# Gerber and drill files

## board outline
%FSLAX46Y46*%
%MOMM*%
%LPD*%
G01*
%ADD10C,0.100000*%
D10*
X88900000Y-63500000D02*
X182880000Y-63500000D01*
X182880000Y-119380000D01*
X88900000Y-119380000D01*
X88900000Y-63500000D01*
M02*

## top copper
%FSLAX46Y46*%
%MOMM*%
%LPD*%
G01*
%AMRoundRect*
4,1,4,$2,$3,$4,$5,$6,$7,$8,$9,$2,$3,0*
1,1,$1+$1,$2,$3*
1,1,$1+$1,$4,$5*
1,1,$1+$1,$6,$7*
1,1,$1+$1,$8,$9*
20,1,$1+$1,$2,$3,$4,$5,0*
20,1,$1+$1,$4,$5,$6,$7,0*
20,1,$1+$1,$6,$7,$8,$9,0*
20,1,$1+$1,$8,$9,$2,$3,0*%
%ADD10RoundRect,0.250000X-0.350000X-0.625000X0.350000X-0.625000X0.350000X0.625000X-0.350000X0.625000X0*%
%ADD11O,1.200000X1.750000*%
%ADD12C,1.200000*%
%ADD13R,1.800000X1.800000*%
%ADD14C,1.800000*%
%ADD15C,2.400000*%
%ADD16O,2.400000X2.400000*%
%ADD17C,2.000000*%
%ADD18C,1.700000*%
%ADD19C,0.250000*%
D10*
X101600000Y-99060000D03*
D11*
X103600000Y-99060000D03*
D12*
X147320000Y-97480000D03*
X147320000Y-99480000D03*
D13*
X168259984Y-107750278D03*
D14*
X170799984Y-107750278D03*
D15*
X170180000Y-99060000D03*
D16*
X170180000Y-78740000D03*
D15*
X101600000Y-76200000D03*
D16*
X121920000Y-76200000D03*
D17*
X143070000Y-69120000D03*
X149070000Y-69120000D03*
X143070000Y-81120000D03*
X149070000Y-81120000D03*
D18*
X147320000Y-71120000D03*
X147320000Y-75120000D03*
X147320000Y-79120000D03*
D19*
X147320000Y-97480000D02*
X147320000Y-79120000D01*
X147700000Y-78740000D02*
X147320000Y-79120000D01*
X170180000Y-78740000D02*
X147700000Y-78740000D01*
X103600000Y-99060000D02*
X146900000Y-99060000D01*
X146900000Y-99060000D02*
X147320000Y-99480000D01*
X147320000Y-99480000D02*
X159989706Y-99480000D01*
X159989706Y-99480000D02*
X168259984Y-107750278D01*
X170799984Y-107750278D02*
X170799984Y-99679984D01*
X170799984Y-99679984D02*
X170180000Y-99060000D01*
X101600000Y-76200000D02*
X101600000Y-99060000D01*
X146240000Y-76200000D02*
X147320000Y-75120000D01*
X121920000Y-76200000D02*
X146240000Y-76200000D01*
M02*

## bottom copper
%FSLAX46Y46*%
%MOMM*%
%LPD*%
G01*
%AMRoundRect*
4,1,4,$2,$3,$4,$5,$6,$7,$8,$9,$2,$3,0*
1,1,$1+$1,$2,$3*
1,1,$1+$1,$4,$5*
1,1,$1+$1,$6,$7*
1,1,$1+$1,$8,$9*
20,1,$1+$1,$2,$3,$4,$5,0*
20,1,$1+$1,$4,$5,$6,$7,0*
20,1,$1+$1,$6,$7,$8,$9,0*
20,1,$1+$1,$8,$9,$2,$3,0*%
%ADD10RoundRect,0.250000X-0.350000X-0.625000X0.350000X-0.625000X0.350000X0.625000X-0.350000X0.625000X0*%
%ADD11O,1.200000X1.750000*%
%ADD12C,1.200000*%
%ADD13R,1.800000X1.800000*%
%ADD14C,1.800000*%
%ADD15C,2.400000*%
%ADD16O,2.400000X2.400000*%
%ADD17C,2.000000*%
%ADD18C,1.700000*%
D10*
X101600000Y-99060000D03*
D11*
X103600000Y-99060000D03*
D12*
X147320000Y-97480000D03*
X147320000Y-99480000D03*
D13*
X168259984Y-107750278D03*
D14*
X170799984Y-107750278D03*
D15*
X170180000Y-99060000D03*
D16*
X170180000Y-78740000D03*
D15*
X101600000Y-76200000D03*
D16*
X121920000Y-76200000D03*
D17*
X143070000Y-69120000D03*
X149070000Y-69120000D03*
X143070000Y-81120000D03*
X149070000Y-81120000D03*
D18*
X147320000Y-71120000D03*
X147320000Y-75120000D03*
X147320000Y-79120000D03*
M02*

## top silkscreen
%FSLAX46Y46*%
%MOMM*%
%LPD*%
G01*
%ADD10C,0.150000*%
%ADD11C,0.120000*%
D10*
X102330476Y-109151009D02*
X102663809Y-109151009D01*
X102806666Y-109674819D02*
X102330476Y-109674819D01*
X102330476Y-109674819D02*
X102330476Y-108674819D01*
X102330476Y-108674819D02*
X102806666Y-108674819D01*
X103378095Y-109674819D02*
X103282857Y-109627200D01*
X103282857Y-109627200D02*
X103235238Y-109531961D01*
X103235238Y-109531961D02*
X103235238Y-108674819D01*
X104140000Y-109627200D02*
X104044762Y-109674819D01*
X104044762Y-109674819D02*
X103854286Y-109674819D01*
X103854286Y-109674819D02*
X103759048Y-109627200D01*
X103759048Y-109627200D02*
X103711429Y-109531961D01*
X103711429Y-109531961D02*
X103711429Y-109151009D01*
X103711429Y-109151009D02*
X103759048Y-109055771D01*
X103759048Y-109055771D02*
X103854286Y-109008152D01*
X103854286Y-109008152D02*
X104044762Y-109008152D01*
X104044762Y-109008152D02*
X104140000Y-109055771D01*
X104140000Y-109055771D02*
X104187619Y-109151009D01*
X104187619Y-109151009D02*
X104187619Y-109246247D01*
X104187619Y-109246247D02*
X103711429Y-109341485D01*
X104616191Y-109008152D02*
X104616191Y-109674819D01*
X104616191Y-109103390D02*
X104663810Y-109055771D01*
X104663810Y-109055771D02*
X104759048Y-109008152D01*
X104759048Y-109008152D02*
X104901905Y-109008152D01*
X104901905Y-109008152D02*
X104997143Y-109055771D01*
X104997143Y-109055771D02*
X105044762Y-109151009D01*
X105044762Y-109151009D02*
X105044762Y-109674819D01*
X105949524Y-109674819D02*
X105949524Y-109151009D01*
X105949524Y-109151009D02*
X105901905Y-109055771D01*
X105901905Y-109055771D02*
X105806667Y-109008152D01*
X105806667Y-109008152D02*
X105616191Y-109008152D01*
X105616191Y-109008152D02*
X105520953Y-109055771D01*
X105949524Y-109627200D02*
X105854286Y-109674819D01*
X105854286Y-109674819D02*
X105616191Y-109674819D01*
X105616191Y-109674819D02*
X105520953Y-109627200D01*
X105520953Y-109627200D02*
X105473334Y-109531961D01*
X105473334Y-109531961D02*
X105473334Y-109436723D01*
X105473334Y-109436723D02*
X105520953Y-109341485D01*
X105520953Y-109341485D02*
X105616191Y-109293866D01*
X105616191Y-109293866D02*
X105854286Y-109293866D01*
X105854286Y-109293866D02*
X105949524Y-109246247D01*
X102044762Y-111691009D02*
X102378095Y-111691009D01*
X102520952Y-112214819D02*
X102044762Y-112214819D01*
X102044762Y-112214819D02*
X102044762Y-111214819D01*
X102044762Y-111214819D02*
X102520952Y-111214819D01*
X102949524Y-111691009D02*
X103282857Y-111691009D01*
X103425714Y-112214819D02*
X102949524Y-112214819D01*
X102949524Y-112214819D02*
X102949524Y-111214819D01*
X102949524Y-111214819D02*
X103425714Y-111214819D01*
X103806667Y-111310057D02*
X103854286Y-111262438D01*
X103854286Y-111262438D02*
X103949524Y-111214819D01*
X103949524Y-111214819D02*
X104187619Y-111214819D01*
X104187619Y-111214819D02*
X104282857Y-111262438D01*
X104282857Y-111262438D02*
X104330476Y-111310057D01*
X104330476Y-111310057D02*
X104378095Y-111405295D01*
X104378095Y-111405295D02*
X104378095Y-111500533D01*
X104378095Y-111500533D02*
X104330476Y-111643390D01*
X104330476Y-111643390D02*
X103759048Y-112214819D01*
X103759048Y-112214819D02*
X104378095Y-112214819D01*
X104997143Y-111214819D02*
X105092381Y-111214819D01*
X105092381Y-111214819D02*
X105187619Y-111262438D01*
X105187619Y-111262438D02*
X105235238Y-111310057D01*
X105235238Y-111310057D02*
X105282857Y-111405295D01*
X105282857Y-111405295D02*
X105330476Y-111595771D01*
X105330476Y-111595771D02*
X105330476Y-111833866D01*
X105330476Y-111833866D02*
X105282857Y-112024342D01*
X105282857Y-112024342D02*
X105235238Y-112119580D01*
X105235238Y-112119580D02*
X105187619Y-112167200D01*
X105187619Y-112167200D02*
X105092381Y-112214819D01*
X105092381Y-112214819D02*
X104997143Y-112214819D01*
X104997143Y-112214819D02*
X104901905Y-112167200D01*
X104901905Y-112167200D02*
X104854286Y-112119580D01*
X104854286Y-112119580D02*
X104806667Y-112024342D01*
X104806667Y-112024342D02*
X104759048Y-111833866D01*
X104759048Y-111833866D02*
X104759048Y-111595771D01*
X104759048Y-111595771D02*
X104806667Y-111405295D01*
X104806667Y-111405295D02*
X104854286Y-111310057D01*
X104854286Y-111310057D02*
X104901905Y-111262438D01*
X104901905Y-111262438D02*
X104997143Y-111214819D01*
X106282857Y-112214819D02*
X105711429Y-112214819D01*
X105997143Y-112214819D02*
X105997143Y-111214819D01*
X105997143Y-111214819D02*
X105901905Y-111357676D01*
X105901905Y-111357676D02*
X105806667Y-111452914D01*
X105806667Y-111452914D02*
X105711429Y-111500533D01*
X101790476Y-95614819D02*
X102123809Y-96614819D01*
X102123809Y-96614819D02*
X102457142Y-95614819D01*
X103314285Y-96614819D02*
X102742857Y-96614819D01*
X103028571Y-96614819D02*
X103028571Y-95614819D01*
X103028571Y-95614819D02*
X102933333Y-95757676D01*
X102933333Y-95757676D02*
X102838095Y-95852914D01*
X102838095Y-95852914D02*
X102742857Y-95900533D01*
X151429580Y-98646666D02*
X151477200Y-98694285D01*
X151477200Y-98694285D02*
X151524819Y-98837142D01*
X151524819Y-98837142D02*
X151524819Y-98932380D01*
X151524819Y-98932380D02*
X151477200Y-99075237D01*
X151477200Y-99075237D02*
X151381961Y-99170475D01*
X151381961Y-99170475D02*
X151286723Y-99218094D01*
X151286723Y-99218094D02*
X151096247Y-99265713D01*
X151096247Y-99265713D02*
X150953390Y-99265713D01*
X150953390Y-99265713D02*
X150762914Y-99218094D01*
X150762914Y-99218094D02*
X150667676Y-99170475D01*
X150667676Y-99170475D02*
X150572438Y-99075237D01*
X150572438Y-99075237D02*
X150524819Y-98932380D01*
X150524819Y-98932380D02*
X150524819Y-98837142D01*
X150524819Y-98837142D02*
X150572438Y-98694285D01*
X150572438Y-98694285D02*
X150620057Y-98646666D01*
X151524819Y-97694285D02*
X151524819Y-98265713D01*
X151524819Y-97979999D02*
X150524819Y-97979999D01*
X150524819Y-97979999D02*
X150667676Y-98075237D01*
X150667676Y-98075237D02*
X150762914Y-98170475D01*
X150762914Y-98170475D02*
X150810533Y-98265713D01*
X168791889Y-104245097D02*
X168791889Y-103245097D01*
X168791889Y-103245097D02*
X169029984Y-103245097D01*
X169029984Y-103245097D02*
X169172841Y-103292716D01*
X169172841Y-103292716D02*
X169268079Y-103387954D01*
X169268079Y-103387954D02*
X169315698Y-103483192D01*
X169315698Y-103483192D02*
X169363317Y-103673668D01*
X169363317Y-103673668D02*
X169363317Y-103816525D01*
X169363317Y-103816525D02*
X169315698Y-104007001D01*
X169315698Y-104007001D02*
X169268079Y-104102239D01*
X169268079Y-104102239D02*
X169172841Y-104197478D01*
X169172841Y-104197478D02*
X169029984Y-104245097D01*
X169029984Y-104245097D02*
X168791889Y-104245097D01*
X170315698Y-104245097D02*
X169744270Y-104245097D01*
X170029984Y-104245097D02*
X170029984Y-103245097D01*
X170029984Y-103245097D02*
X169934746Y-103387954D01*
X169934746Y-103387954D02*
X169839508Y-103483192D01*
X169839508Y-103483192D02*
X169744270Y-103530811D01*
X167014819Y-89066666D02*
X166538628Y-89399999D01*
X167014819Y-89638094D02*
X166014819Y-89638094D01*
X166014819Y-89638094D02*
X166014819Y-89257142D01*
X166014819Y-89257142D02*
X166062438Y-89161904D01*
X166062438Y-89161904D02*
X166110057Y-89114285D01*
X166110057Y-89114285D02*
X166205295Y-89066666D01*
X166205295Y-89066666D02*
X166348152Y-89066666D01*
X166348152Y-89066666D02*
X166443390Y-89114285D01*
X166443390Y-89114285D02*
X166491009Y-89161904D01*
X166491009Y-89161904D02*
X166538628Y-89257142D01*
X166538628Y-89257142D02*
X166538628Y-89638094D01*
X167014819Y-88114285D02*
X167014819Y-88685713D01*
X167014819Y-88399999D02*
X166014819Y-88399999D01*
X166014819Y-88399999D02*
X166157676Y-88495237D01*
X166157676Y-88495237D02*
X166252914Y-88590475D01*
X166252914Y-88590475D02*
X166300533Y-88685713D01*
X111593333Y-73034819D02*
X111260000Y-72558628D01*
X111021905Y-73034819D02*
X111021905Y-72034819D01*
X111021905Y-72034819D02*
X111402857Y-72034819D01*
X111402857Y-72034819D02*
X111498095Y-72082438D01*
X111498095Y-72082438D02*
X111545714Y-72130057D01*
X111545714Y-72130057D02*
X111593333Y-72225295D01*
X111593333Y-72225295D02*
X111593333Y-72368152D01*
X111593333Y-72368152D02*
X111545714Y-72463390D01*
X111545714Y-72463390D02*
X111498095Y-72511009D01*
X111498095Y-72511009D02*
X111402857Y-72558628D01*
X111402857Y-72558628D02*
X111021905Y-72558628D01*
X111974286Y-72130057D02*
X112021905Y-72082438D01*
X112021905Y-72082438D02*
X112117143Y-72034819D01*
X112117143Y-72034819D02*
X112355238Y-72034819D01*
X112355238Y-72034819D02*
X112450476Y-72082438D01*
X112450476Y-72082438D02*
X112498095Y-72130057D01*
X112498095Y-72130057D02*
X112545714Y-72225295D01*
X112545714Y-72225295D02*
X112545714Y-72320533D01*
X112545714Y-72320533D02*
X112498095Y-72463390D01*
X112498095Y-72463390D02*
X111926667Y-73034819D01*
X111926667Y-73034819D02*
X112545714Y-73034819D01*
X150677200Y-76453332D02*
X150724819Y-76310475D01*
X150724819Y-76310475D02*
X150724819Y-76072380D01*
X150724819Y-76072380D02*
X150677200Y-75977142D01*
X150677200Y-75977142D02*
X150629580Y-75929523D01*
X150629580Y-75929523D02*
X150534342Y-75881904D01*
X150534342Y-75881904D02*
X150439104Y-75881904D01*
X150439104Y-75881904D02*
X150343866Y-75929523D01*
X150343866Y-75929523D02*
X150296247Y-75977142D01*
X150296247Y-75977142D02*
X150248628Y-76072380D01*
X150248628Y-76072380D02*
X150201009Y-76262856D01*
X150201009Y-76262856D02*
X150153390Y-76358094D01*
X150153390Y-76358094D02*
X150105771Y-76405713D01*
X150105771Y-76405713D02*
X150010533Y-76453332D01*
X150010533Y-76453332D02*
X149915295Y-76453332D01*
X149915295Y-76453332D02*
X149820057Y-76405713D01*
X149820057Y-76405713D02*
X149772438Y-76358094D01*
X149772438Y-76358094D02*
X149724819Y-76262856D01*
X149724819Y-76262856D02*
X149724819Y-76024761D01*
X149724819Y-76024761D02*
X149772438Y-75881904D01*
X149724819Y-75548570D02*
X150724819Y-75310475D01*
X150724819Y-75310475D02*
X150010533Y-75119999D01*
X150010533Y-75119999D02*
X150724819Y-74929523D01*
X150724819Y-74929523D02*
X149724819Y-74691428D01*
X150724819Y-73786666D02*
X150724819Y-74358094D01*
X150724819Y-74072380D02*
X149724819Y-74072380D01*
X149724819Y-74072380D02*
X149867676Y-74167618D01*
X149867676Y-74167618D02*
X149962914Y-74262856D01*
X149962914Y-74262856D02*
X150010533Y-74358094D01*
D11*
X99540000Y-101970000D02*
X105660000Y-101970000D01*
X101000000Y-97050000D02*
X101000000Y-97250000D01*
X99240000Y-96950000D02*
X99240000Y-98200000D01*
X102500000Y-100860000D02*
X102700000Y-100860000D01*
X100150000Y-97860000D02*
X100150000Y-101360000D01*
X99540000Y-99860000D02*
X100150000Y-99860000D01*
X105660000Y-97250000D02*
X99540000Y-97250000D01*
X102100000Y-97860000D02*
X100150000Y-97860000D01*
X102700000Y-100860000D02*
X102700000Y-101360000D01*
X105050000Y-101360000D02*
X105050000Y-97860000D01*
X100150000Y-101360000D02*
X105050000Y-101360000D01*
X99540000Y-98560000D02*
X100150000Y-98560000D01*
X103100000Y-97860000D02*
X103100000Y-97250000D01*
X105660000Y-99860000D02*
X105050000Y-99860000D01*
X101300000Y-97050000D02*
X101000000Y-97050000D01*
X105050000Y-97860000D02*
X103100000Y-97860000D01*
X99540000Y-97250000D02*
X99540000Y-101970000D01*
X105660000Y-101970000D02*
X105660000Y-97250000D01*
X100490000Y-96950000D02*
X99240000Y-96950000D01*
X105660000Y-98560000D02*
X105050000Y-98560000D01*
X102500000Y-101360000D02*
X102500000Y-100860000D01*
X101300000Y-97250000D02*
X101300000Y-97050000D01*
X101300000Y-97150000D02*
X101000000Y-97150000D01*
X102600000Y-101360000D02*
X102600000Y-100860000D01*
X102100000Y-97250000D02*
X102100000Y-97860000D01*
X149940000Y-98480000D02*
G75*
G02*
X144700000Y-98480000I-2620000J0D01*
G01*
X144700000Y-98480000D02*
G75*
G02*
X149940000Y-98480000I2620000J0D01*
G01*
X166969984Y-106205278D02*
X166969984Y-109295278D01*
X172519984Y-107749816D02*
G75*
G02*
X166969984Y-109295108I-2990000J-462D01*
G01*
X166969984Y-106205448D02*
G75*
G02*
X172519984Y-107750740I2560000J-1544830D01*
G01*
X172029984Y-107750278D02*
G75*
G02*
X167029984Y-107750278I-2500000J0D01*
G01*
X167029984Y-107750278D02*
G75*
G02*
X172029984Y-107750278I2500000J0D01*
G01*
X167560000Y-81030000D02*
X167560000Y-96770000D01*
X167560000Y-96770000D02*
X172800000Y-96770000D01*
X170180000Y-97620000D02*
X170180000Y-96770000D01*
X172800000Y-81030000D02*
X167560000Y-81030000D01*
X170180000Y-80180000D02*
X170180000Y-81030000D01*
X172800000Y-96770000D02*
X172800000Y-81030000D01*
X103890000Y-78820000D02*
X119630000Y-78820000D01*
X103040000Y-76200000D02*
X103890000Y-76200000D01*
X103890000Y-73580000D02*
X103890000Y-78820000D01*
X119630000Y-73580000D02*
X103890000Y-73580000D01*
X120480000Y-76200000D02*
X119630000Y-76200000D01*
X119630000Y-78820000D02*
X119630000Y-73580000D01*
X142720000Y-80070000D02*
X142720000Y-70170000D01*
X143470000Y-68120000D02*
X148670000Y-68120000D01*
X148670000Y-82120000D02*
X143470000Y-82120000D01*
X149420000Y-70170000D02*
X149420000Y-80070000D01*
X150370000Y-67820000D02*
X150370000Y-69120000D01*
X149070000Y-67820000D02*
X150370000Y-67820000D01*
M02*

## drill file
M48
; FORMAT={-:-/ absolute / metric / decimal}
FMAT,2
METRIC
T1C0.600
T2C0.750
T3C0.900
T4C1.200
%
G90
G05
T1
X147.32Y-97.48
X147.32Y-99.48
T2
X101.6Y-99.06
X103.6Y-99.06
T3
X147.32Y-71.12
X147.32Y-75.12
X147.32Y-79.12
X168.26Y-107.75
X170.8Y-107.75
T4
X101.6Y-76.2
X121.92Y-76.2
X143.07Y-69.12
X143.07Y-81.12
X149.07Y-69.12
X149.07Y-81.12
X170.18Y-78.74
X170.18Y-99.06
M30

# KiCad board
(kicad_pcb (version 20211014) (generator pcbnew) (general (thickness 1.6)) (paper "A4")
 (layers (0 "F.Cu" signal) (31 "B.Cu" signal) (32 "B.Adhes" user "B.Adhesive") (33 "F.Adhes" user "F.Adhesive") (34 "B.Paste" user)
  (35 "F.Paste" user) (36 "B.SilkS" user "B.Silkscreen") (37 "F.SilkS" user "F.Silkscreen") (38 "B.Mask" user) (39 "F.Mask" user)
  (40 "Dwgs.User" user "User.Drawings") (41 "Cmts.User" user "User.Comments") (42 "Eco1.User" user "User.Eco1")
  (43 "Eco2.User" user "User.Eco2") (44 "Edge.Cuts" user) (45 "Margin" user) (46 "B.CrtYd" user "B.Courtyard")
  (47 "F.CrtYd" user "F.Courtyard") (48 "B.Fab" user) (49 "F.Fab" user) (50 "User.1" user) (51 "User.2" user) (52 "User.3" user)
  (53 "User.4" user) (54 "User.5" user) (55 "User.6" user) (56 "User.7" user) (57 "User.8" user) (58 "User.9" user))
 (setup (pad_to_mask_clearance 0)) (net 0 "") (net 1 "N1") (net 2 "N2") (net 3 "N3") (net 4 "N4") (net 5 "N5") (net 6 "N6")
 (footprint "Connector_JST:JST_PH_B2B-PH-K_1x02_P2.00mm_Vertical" (layer "F.Cu") (at 101.6 99.06)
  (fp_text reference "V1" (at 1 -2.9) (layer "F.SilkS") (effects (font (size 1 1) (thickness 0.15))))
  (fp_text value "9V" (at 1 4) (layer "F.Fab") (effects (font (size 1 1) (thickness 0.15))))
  (fp_line (start -2.06 2.91) (end 4.06 2.91) (layer "F.SilkS") (width 0.12))
  (fp_line (start -0.6 -2.01) (end -0.6 -1.81) (layer "F.SilkS") (width 0.12))
  (fp_line (start -2.36 -2.11) (end -2.36 -0.86) (layer "F.SilkS") (width 0.12))
  (fp_line (start 0.9 1.8) (end 1.1 1.8) (layer "F.SilkS") (width 0.12))
  (fp_line (start -1.45 -1.2) (end -1.45 2.3) (layer "F.SilkS") (width 0.12))
  (fp_line (start -2.06 0.8) (end -1.45 0.8) (layer "F.SilkS") (width 0.12))
  (fp_line (start 4.06 -1.81) (end -2.06 -1.81) (layer "F.SilkS") (width 0.12))
  (fp_line (start 0.5 -1.2) (end -1.45 -1.2) (layer "F.SilkS") (width 0.12))
  (fp_line (start 1.1 1.8) (end 1.1 2.3) (layer "F.SilkS") (width 0.12))
  (fp_line (start 3.45 2.3) (end 3.45 -1.2) (layer "F.SilkS") (width 0.12))
  (fp_line (start -1.45 2.3) (end 3.45 2.3) (layer "F.SilkS") (width 0.12))
  (fp_line (start -2.06 -0.5) (end -1.45 -0.5) (layer "F.SilkS") (width 0.12))
  (fp_line (start 1.5 -1.2) (end 1.5 -1.81) (layer "F.SilkS") (width 0.12))
  (fp_line (start 4.06 0.8) (end 3.45 0.8) (layer "F.SilkS") (width 0.12))
  (fp_line (start -0.3 -2.01) (end -0.6 -2.01) (layer "F.SilkS") (width 0.12))
  (fp_line (start 3.45 -1.2) (end 1.5 -1.2) (layer "F.SilkS") (width 0.12))
  (fp_line (start -2.06 -1.81) (end -2.06 2.91) (layer "F.SilkS") (width 0.12))
  (fp_line (start 4.06 2.91) (end 4.06 -1.81) (layer "F.SilkS") (width 0.12))
  (fp_line (start -1.11 -2.11) (end -2.36 -2.11) (layer "F.SilkS") (width 0.12))
  (fp_line (start 4.06 -0.5) (end 3.45 -0.5) (layer "F.SilkS") (width 0.12))
  (fp_line (start 0.9 2.3) (end 0.9 1.8) (layer "F.SilkS") (width 0.12))
  (fp_line (start -0.3 -1.81) (end -0.3 -2.01) (layer "F.SilkS") (width 0.12))
  (fp_line (start -0.3 -1.91) (end -0.6 -1.91) (layer "F.SilkS") (width 0.12))
  (fp_line (start 1 2.3) (end 1 1.8) (layer "F.SilkS") (width 0.12))
  (fp_line (start 0.5 -1.81) (end 0.5 -1.2) (layer "F.SilkS") (width 0.12))
  (pad "1" thru_hole roundrect (at 0 0) (size 1.2 1.75) (drill 0.75) (layers *.Cu *.Mask) (roundrect_rratio 0.208333) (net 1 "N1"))
  (pad "2" thru_hole oval (at 2 0) (size 1.2 1.75) (drill 0.75) (layers *.Cu *.Mask) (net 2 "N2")))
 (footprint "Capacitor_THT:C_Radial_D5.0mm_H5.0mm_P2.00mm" (layer "F.Cu") (at 147.32 97.48 -90)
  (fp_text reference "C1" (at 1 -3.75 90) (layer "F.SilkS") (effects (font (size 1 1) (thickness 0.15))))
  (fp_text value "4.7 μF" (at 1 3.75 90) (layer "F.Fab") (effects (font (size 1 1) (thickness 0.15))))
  (fp_circle (center 1 0) (end 3.62 0) (layer "F.SilkS") (width 0.12) (fill none))
  (pad "1" thru_hole circle (at 0 0 270) (size 1.2 1.2) (drill 0.6) (layers *.Cu *.Mask) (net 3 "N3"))
  (pad "2" thru_hole circle (at 2 0 270) (size 1.2 1.2) (drill 0.6) (layers *.Cu *.Mask) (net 2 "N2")))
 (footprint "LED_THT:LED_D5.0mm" (layer "F.Cu") (at 168.259984 107.750278)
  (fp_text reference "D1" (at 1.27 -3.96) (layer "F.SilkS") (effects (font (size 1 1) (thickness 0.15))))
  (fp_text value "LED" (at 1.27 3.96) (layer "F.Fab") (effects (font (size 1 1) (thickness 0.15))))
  (fp_line (start -1.29 -1.545) (end -1.29 1.545) (layer "F.SilkS") (width 0.12))
  (fp_arc (start 4.26 -0.000462) (mid 2.072002 2.880433) (end -1.29 1.54483) (layer "F.SilkS") (width 0.12))
  (fp_arc (start -1.29 -1.54483) (mid 2.072002 -2.880433) (end 4.26 0.000462) (layer "F.SilkS") (width 0.12))
  (fp_circle (center 1.27 0) (end 3.77 0) (layer "F.SilkS") (width 0.12) (fill none))
  (pad "1" thru_hole rect (at 0 0) (size 1.8 1.8) (drill 0.9) (layers *.Cu *.Mask) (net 2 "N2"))
  (pad "2" thru_hole circle (at 2.54 0) (size 1.8 1.8) (drill 0.9) (layers *.Cu *.Mask) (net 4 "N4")))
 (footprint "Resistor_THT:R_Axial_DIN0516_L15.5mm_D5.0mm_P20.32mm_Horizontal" (layer "F.Cu") (at 170.18 99.06 90)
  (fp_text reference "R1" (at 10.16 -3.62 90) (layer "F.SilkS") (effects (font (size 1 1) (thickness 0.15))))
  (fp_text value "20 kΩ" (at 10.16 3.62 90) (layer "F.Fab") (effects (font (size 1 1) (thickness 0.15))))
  (fp_line (start 18.03 -2.62) (end 2.29 -2.62) (layer "F.SilkS") (width 0.12))
  (fp_line (start 2.29 -2.62) (end 2.29 2.62) (layer "F.SilkS") (width 0.12))
  (fp_line (start 1.44 0) (end 2.29 0) (layer "F.SilkS") (width 0.12))
  (fp_line (start 18.03 2.62) (end 18.03 -2.62) (layer "F.SilkS") (width 0.12))
  (fp_line (start 18.88 0) (end 18.03 0) (layer "F.SilkS") (width 0.12))
  (fp_line (start 2.29 2.62) (end 18.03 2.62) (layer "F.SilkS") (width 0.12))
  (pad "1" thru_hole circle (at 0 0 90) (size 2.4 2.4) (drill 1.2) (layers *.Cu *.Mask) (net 4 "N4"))
  (pad "2" thru_hole oval (at 20.32 0 90) (size 2.4 2.4) (drill 1.2) (layers *.Cu *.Mask) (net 3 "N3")))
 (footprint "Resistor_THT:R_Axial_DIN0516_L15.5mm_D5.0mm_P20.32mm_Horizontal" (layer "F.Cu") (at 101.6 76.2)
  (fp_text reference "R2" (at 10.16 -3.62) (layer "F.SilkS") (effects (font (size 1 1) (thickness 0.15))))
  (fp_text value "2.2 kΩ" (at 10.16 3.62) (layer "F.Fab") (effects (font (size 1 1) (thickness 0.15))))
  (fp_line (start 2.29 2.62) (end 18.03 2.62) (layer "F.SilkS") (width 0.12))
  (fp_line (start 1.44 0) (end 2.29 0) (layer "F.SilkS") (width 0.12))
  (fp_line (start 2.29 -2.62) (end 2.29 2.62) (layer "F.SilkS") (width 0.12))
  (fp_line (start 18.03 -2.62) (end 2.29 -2.62) (layer "F.SilkS") (width 0.12))
  (fp_line (start 18.88 0) (end 18.03 0) (layer "F.SilkS") (width 0.12))
  (fp_line (start 18.03 2.62) (end 18.03 -2.62) (layer "F.SilkS") (width 0.12))
  (pad "1" thru_hole circle (at 0 0) (size 2.4 2.4) (drill 1.2) (layers *.Cu *.Mask) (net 1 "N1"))
  (pad "2" thru_hole oval (at 20.32 0) (size 2.4 2.4) (drill 1.2) (layers *.Cu *.Mask) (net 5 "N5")))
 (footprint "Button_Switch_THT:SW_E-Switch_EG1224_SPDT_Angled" (layer "F.Cu") (at 147.32 71.12 -90)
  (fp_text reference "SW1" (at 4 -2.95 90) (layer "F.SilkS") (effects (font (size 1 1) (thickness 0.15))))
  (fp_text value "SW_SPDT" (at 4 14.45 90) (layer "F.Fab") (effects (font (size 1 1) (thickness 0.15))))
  (fp_line (start 8.95 4.6) (end -0.95 4.6) (layer "F.SilkS") (width 0.12))
  (fp_line (start -3 3.85) (end -3 -1.35) (layer "F.SilkS") (width 0.12))
  (fp_line (start 11 -1.35) (end 11 3.85) (layer "F.SilkS") (width 0.12))
  (fp_line (start -0.95 -2.1) (end 8.95 -2.1) (layer "F.SilkS") (width 0.12))
  (fp_line (start -3.3 -3.05) (end -2 -3.05) (layer "F.SilkS") (width 0.12))
  (fp_line (start -3.3 -1.75) (end -3.3 -3.05) (layer "F.SilkS") (width 0.12))
  (pad "" thru_hole circle (at -2 4.25 270) (size 2 2) (drill 1.2) (layers *.Cu *.Mask))
  (pad "" thru_hole circle (at -2 -1.75 270) (size 2 2) (drill 1.2) (layers *.Cu *.Mask))
  (pad "" thru_hole circle (at 10 4.25 270) (size 2 2) (drill 1.2) (layers *.Cu *.Mask))
  (pad "" thru_hole circle (at 10 -1.75 270) (size 2 2) (drill 1.2) (layers *.Cu *.Mask))
  (pad "1" thru_hole circle (at 0 0 270) (size 1.7 1.7) (drill 0.9) (layers *.Cu *.Mask) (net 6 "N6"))
  (pad "2" thru_hole circle (at 4 0 270) (size 1.7 1.7) (drill 0.9) (layers *.Cu *.Mask) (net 5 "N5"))
  (pad "3" thru_hole circle (at 8 0 270) (size 1.7 1.7) (drill 0.9) (layers *.Cu *.Mask) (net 3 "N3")))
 (gr_rect (start 88.9 63.5) (end 182.88 119.38) (layer "Edge.Cuts") (width 0.1) (fill none))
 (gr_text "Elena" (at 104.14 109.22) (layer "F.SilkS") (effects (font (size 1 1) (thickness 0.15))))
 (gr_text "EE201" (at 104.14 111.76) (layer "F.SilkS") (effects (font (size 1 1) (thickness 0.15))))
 (segment (start 147.32 97.48) (end 147.32 79.12) (width 0.25) (layer "F.Cu") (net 3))
 (segment (start 147.7 78.74) (end 147.32 79.12) (width 0.25) (layer "F.Cu") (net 3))
 (segment (start 170.18 78.74) (end 147.7 78.74) (width 0.25) (layer "F.Cu") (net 3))
 (segment (start 103.6 99.06) (end 146.9 99.06) (width 0.25) (layer "F.Cu") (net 2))
 (segment (start 146.9 99.06) (end 147.32 99.48) (width 0.25) (layer "F.Cu") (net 2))
 (segment (start 147.32 99.48) (end 159.989706 99.48) (width 0.25) (layer "F.Cu") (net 2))
 (segment (start 159.989706 99.48) (end 168.259984 107.750278) (width 0.25) (layer "F.Cu") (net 2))
 (segment (start 170.799984 107.750278) (end 170.799984 99.679984) (width 0.25) (layer "F.Cu") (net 4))
 (segment (start 170.799984 99.679984) (end 170.18 99.06) (width 0.25) (layer "F.Cu") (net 4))
 (segment (start 101.6 76.2) (end 101.6 99.06) (width 0.25) (layer "F.Cu") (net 1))
 (segment (start 146.24 76.2) (end 147.32 75.12) (width 0.25) (layer "F.Cu") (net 5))
 (segment (start 121.92 76.2) (end 146.24 76.2) (width 0.25) (layer "F.Cu") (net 5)))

